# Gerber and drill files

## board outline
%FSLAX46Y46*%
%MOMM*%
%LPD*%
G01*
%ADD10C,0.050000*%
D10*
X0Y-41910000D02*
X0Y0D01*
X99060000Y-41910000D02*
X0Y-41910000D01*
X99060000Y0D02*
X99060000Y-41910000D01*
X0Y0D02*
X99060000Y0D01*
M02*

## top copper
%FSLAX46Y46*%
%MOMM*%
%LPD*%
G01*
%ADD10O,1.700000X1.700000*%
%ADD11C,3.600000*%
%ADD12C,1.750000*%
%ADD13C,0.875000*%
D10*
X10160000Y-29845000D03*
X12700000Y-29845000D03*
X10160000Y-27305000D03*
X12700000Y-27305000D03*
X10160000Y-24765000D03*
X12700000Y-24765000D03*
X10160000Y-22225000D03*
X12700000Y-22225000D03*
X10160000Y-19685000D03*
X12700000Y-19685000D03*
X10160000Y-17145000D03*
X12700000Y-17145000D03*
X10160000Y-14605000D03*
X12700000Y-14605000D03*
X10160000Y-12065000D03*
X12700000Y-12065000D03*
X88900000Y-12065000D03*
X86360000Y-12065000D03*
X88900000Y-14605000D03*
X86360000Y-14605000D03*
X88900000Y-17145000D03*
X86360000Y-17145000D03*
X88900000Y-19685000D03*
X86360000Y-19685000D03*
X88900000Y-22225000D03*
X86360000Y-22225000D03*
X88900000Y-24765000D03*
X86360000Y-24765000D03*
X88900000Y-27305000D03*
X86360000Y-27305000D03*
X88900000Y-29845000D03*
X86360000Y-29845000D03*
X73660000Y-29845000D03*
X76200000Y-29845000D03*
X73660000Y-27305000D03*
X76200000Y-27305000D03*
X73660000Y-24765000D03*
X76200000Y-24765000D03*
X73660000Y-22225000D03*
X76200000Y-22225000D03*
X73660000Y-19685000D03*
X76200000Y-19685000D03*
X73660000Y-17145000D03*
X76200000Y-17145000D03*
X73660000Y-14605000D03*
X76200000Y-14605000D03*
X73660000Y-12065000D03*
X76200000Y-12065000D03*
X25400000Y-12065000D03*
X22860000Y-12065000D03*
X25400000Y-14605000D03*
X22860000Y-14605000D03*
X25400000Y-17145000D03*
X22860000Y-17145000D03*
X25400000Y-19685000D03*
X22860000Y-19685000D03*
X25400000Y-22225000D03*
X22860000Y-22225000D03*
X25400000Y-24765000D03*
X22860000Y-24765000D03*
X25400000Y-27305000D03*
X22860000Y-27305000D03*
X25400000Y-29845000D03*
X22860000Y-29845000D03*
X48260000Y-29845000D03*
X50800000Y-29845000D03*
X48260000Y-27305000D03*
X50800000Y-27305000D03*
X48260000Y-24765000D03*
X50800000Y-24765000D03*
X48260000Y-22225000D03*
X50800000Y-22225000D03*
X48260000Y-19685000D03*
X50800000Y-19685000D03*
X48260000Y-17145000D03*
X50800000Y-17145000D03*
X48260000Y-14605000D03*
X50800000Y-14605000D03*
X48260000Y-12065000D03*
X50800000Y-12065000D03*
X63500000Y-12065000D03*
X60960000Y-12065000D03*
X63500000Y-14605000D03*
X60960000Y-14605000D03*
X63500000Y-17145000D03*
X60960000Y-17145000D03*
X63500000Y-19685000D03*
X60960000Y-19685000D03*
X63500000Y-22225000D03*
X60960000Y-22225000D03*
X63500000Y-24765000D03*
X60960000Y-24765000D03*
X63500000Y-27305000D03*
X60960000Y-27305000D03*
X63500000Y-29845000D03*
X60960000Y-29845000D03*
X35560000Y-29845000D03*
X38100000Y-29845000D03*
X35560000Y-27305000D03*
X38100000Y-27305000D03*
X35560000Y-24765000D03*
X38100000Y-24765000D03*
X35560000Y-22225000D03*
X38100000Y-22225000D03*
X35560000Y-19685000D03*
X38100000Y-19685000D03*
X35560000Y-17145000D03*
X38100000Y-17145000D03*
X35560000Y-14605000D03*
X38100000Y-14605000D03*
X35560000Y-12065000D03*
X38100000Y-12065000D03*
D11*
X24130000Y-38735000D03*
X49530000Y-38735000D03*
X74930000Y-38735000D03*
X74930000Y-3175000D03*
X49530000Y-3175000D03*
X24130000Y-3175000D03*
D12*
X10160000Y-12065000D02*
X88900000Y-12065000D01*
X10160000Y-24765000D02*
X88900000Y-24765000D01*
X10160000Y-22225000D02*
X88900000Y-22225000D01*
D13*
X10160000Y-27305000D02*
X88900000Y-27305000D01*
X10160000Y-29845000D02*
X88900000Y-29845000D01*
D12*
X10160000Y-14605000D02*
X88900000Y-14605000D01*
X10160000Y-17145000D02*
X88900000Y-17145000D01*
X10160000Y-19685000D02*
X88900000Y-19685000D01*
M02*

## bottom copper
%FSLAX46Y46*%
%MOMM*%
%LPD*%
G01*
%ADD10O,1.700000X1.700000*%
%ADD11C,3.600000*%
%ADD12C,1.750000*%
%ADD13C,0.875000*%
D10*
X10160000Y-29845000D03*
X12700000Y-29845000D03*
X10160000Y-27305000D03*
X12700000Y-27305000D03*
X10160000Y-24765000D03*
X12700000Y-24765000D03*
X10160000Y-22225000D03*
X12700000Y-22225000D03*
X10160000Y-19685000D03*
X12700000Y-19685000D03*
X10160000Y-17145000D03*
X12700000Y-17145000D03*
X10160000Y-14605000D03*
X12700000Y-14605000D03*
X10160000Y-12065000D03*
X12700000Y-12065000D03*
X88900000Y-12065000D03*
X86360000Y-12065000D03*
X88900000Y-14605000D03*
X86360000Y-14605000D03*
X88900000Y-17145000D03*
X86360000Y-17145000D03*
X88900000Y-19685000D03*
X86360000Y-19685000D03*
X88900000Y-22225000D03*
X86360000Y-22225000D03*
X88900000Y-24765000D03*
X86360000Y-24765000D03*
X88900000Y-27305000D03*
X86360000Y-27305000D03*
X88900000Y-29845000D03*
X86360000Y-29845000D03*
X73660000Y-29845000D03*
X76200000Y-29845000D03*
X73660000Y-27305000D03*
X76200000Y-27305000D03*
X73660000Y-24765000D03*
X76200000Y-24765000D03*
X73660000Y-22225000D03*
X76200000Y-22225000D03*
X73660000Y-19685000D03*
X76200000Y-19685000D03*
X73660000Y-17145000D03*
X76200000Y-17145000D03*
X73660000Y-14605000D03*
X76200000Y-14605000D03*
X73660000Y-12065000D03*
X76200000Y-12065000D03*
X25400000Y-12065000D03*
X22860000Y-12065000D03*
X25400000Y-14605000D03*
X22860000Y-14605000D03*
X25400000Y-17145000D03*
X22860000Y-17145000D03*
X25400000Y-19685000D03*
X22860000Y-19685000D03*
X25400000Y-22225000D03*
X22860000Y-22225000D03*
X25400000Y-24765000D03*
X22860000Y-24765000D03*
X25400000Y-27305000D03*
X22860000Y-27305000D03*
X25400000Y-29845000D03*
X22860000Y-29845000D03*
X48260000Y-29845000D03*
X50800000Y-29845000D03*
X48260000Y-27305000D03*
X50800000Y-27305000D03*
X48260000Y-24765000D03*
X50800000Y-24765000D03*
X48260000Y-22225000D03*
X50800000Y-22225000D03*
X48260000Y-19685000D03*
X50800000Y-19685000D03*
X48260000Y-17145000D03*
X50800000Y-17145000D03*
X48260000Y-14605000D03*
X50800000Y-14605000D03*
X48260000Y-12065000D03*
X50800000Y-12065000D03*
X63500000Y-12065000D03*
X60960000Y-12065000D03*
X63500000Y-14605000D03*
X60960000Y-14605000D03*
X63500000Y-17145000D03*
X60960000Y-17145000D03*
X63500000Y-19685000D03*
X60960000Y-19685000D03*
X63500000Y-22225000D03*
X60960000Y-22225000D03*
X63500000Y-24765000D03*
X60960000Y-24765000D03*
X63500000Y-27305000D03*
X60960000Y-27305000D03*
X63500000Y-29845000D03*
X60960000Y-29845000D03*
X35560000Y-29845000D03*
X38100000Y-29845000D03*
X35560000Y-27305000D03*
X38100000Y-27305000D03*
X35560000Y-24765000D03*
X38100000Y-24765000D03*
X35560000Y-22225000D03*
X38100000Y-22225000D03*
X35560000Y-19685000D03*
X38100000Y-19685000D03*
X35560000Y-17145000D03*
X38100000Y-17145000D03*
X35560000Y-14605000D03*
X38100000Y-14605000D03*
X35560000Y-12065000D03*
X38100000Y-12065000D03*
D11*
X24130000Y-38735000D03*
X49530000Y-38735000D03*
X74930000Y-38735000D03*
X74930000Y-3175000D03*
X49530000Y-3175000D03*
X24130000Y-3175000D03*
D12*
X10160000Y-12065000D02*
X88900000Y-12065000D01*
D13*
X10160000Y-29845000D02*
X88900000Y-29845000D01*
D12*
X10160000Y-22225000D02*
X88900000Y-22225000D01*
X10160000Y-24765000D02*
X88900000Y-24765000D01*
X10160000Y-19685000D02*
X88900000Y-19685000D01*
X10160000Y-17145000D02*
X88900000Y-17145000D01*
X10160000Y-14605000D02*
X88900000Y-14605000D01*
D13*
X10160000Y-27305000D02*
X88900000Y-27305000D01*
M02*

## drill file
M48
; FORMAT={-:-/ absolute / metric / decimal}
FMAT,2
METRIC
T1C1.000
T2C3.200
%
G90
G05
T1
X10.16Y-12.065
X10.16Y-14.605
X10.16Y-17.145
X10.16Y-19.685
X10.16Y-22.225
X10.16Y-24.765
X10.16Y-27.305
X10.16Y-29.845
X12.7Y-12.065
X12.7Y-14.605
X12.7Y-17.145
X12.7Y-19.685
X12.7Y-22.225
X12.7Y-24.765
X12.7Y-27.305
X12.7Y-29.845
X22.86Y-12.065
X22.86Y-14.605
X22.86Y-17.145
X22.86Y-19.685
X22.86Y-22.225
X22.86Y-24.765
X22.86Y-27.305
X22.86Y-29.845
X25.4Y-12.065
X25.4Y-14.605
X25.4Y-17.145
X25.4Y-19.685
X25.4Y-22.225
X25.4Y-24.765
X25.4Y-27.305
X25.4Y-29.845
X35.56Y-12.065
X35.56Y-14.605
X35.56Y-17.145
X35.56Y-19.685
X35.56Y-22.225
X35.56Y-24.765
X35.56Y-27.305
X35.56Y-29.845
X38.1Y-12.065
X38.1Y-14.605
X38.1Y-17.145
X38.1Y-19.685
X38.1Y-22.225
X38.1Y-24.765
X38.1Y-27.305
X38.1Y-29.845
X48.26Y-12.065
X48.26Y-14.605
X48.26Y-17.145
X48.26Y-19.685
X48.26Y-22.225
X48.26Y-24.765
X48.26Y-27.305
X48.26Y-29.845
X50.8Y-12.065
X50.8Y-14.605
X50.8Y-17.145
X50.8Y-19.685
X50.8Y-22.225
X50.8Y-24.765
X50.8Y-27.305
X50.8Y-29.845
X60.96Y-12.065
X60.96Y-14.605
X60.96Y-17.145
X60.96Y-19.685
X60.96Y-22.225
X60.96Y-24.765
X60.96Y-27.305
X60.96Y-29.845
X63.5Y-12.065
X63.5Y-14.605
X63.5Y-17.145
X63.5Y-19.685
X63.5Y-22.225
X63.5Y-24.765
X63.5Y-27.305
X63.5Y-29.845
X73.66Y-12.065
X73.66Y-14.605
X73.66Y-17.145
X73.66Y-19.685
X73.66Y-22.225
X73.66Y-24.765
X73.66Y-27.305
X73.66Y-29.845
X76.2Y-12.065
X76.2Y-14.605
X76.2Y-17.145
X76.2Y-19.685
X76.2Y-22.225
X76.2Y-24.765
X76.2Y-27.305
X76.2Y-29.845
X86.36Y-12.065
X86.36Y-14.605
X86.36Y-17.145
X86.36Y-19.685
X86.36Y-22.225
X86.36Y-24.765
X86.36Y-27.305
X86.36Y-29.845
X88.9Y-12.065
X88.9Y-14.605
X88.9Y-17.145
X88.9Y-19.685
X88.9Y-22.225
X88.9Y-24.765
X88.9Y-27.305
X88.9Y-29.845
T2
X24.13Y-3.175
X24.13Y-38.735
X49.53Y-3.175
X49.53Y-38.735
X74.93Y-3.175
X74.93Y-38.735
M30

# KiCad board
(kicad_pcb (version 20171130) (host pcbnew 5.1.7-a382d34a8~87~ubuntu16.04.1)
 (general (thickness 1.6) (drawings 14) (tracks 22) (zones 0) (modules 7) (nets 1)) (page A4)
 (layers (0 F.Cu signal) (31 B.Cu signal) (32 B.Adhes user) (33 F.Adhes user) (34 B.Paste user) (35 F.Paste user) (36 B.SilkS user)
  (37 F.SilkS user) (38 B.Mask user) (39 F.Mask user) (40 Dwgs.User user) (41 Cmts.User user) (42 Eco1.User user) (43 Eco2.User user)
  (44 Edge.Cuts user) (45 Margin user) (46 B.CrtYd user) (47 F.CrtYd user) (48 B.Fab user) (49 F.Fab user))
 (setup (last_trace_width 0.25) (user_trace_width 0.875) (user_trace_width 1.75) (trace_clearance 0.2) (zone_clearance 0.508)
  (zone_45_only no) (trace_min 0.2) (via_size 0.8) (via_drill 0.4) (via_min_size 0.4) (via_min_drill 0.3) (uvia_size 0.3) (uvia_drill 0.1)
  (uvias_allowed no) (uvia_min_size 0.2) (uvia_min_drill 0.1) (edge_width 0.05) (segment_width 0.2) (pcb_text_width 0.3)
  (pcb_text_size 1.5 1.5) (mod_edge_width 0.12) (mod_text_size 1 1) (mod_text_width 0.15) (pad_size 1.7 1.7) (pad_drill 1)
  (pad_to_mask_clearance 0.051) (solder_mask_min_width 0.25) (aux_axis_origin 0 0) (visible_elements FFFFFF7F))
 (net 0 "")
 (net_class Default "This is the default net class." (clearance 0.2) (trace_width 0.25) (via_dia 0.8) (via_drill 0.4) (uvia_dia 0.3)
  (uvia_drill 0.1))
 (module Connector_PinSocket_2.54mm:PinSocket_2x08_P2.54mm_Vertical (layer F.Cu) (at 12.7 12.065)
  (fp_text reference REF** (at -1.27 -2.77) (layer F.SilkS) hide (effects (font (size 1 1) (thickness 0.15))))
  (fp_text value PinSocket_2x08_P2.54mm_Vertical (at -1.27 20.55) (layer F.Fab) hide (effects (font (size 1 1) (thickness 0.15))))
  (pad 16 thru_hole oval (at -2.54 17.78) (size 1.7 1.7) (drill 1) (layers *.Cu *.Mask))
  (pad 15 thru_hole oval (at 0 17.78) (size 1.7 1.7) (drill 1) (layers *.Cu *.Mask))
  (pad 14 thru_hole oval (at -2.54 15.24) (size 1.7 1.7) (drill 1) (layers *.Cu *.Mask))
  (pad 13 thru_hole oval (at 0 15.24) (size 1.7 1.7) (drill 1) (layers *.Cu *.Mask))
  (pad 12 thru_hole oval (at -2.54 12.7) (size 1.7 1.7) (drill 1) (layers *.Cu *.Mask))
  (pad 11 thru_hole oval (at 0 12.7) (size 1.7 1.7) (drill 1) (layers *.Cu *.Mask))
  (pad 10 thru_hole oval (at -2.54 10.16) (size 1.7 1.7) (drill 1) (layers *.Cu *.Mask))
  (pad 9 thru_hole oval (at 0 10.16) (size 1.7 1.7) (drill 1) (layers *.Cu *.Mask))
  (pad 8 thru_hole oval (at -2.54 7.62) (size 1.7 1.7) (drill 1) (layers *.Cu *.Mask))
  (pad 7 thru_hole oval (at 0 7.62) (size 1.7 1.7) (drill 1) (layers *.Cu *.Mask))
  (pad 6 thru_hole oval (at -2.54 5.08) (size 1.7 1.7) (drill 1) (layers *.Cu *.Mask))
  (pad 5 thru_hole oval (at 0 5.08) (size 1.7 1.7) (drill 1) (layers *.Cu *.Mask))
  (pad 4 thru_hole oval (at -2.54 2.54) (size 1.7 1.7) (drill 1) (layers *.Cu *.Mask))
  (pad 3 thru_hole oval (at 0 2.54) (size 1.7 1.7) (drill 1) (layers *.Cu *.Mask))
  (pad 2 thru_hole oval (at -2.54 0) (size 1.7 1.7) (drill 1) (layers *.Cu *.Mask))
  (pad 1 thru_hole oval (at 0 0) (size 1.7 1.7) (drill 1) (layers *.Cu *.Mask)))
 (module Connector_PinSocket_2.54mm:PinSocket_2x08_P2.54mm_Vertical (layer F.Cu) (at 88.9 12.065)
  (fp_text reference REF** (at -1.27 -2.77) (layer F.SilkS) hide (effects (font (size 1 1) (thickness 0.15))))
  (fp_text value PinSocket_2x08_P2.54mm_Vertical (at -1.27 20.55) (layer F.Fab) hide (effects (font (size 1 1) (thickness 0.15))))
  (pad 1 thru_hole oval (at 0 0) (size 1.7 1.7) (drill 1) (layers *.Cu *.Mask))
  (pad 2 thru_hole oval (at -2.54 0) (size 1.7 1.7) (drill 1) (layers *.Cu *.Mask))
  (pad 3 thru_hole oval (at 0 2.54) (size 1.7 1.7) (drill 1) (layers *.Cu *.Mask))
  (pad 4 thru_hole oval (at -2.54 2.54) (size 1.7 1.7) (drill 1) (layers *.Cu *.Mask))
  (pad 5 thru_hole oval (at 0 5.08) (size 1.7 1.7) (drill 1) (layers *.Cu *.Mask))
  (pad 6 thru_hole oval (at -2.54 5.08) (size 1.7 1.7) (drill 1) (layers *.Cu *.Mask))
  (pad 7 thru_hole oval (at 0 7.62) (size 1.7 1.7) (drill 1) (layers *.Cu *.Mask))
  (pad 8 thru_hole oval (at -2.54 7.62) (size 1.7 1.7) (drill 1) (layers *.Cu *.Mask))
  (pad 9 thru_hole oval (at 0 10.16) (size 1.7 1.7) (drill 1) (layers *.Cu *.Mask))
  (pad 10 thru_hole oval (at -2.54 10.16) (size 1.7 1.7) (drill 1) (layers *.Cu *.Mask))
  (pad 11 thru_hole oval (at 0 12.7) (size 1.7 1.7) (drill 1) (layers *.Cu *.Mask))
  (pad 12 thru_hole oval (at -2.54 12.7) (size 1.7 1.7) (drill 1) (layers *.Cu *.Mask))
  (pad 13 thru_hole oval (at 0 15.24) (size 1.7 1.7) (drill 1) (layers *.Cu *.Mask))
  (pad 14 thru_hole oval (at -2.54 15.24) (size 1.7 1.7) (drill 1) (layers *.Cu *.Mask))
  (pad 15 thru_hole oval (at 0 17.78) (size 1.7 1.7) (drill 1) (layers *.Cu *.Mask))
  (pad 16 thru_hole oval (at -2.54 17.78) (size 1.7 1.7) (drill 1) (layers *.Cu *.Mask)))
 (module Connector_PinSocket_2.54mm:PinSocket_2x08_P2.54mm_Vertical (layer F.Cu) (at 76.2 12.065)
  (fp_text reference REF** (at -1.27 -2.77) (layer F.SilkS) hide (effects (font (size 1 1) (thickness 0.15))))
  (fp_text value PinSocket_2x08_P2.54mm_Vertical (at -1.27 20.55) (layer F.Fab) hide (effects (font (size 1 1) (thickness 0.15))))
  (pad 16 thru_hole oval (at -2.54 17.78) (size 1.7 1.7) (drill 1) (layers *.Cu *.Mask))
  (pad 15 thru_hole oval (at 0 17.78) (size 1.7 1.7) (drill 1) (layers *.Cu *.Mask))
  (pad 14 thru_hole oval (at -2.54 15.24) (size 1.7 1.7) (drill 1) (layers *.Cu *.Mask))
  (pad 13 thru_hole oval (at 0 15.24) (size 1.7 1.7) (drill 1) (layers *.Cu *.Mask))
  (pad 12 thru_hole oval (at -2.54 12.7) (size 1.7 1.7) (drill 1) (layers *.Cu *.Mask))
  (pad 11 thru_hole oval (at 0 12.7) (size 1.7 1.7) (drill 1) (layers *.Cu *.Mask))
  (pad 10 thru_hole oval (at -2.54 10.16) (size 1.7 1.7) (drill 1) (layers *.Cu *.Mask))
  (pad 9 thru_hole oval (at 0 10.16) (size 1.7 1.7) (drill 1) (layers *.Cu *.Mask))
  (pad 8 thru_hole oval (at -2.54 7.62) (size 1.7 1.7) (drill 1) (layers *.Cu *.Mask))
  (pad 7 thru_hole oval (at 0 7.62) (size 1.7 1.7) (drill 1) (layers *.Cu *.Mask))
  (pad 6 thru_hole oval (at -2.54 5.08) (size 1.7 1.7) (drill 1) (layers *.Cu *.Mask))
  (pad 5 thru_hole oval (at 0 5.08) (size 1.7 1.7) (drill 1) (layers *.Cu *.Mask))
  (pad 4 thru_hole oval (at -2.54 2.54) (size 1.7 1.7) (drill 1) (layers *.Cu *.Mask))
  (pad 3 thru_hole oval (at 0 2.54) (size 1.7 1.7) (drill 1) (layers *.Cu *.Mask))
  (pad 2 thru_hole oval (at -2.54 0) (size 1.7 1.7) (drill 1) (layers *.Cu *.Mask))
  (pad 1 thru_hole oval (at 0 0) (size 1.7 1.7) (drill 1) (layers *.Cu *.Mask)))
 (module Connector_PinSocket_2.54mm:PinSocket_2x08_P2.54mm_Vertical (layer F.Cu) (at 25.4 12.065)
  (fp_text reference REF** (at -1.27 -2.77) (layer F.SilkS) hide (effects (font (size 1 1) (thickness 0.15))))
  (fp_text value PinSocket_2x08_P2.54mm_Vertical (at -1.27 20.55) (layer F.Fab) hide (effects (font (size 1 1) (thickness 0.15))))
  (pad 1 thru_hole oval (at 0 0) (size 1.7 1.7) (drill 1) (layers *.Cu *.Mask))
  (pad 2 thru_hole oval (at -2.54 0) (size 1.7 1.7) (drill 1) (layers *.Cu *.Mask))
  (pad 3 thru_hole oval (at 0 2.54) (size 1.7 1.7) (drill 1) (layers *.Cu *.Mask))
  (pad 4 thru_hole oval (at -2.54 2.54) (size 1.7 1.7) (drill 1) (layers *.Cu *.Mask))
  (pad 5 thru_hole oval (at 0 5.08) (size 1.7 1.7) (drill 1) (layers *.Cu *.Mask))
  (pad 6 thru_hole oval (at -2.54 5.08) (size 1.7 1.7) (drill 1) (layers *.Cu *.Mask))
  (pad 7 thru_hole oval (at 0 7.62) (size 1.7 1.7) (drill 1) (layers *.Cu *.Mask))
  (pad 8 thru_hole oval (at -2.54 7.62) (size 1.7 1.7) (drill 1) (layers *.Cu *.Mask))
  (pad 9 thru_hole oval (at 0 10.16) (size 1.7 1.7) (drill 1) (layers *.Cu *.Mask))
  (pad 10 thru_hole oval (at -2.54 10.16) (size 1.7 1.7) (drill 1) (layers *.Cu *.Mask))
  (pad 11 thru_hole oval (at 0 12.7) (size 1.7 1.7) (drill 1) (layers *.Cu *.Mask))
  (pad 12 thru_hole oval (at -2.54 12.7) (size 1.7 1.7) (drill 1) (layers *.Cu *.Mask))
  (pad 13 thru_hole oval (at 0 15.24) (size 1.7 1.7) (drill 1) (layers *.Cu *.Mask))
  (pad 14 thru_hole oval (at -2.54 15.24) (size 1.7 1.7) (drill 1) (layers *.Cu *.Mask))
  (pad 15 thru_hole oval (at 0 17.78) (size 1.7 1.7) (drill 1) (layers *.Cu *.Mask))
  (pad 16 thru_hole oval (at -2.54 17.78) (size 1.7 1.7) (drill 1) (layers *.Cu *.Mask)))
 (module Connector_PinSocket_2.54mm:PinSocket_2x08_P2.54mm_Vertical (layer F.Cu) (at 50.8 12.065)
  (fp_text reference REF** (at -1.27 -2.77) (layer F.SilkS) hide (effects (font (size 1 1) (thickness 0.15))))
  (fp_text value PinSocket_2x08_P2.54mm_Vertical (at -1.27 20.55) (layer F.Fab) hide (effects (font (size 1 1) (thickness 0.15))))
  (pad 16 thru_hole oval (at -2.54 17.78) (size 1.7 1.7) (drill 1) (layers *.Cu *.Mask))
  (pad 15 thru_hole oval (at 0 17.78) (size 1.7 1.7) (drill 1) (layers *.Cu *.Mask))
  (pad 14 thru_hole oval (at -2.54 15.24) (size 1.7 1.7) (drill 1) (layers *.Cu *.Mask))
  (pad 13 thru_hole oval (at 0 15.24) (size 1.7 1.7) (drill 1) (layers *.Cu *.Mask))
  (pad 12 thru_hole oval (at -2.54 12.7) (size 1.7 1.7) (drill 1) (layers *.Cu *.Mask))
  (pad 11 thru_hole oval (at 0 12.7) (size 1.7 1.7) (drill 1) (layers *.Cu *.Mask))
  (pad 10 thru_hole oval (at -2.54 10.16) (size 1.7 1.7) (drill 1) (layers *.Cu *.Mask))
  (pad 9 thru_hole oval (at 0 10.16) (size 1.7 1.7) (drill 1) (layers *.Cu *.Mask))
  (pad 8 thru_hole oval (at -2.54 7.62) (size 1.7 1.7) (drill 1) (layers *.Cu *.Mask))
  (pad 7 thru_hole oval (at 0 7.62) (size 1.7 1.7) (drill 1) (layers *.Cu *.Mask))
  (pad 6 thru_hole oval (at -2.54 5.08) (size 1.7 1.7) (drill 1) (layers *.Cu *.Mask))
  (pad 5 thru_hole oval (at 0 5.08) (size 1.7 1.7) (drill 1) (layers *.Cu *.Mask))
  (pad 4 thru_hole oval (at -2.54 2.54) (size 1.7 1.7) (drill 1) (layers *.Cu *.Mask))
  (pad 3 thru_hole oval (at 0 2.54) (size 1.7 1.7) (drill 1) (layers *.Cu *.Mask))
  (pad 2 thru_hole oval (at -2.54 0) (size 1.7 1.7) (drill 1) (layers *.Cu *.Mask))
  (pad 1 thru_hole oval (at 0 0) (size 1.7 1.7) (drill 1) (layers *.Cu *.Mask)))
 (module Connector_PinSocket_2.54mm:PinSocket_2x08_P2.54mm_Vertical (layer F.Cu) (at 63.5 12.065)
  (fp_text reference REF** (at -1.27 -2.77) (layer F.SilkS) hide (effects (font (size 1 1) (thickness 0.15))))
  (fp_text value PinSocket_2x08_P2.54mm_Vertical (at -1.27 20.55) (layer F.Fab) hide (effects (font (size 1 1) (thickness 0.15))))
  (pad 1 thru_hole oval (at 0 0) (size 1.7 1.7) (drill 1) (layers *.Cu *.Mask))
  (pad 2 thru_hole oval (at -2.54 0) (size 1.7 1.7) (drill 1) (layers *.Cu *.Mask))
  (pad 3 thru_hole oval (at 0 2.54) (size 1.7 1.7) (drill 1) (layers *.Cu *.Mask))
  (pad 4 thru_hole oval (at -2.54 2.54) (size 1.7 1.7) (drill 1) (layers *.Cu *.Mask))
  (pad 5 thru_hole oval (at 0 5.08) (size 1.7 1.7) (drill 1) (layers *.Cu *.Mask))
  (pad 6 thru_hole oval (at -2.54 5.08) (size 1.7 1.7) (drill 1) (layers *.Cu *.Mask))
  (pad 7 thru_hole oval (at 0 7.62) (size 1.7 1.7) (drill 1) (layers *.Cu *.Mask))
  (pad 8 thru_hole oval (at -2.54 7.62) (size 1.7 1.7) (drill 1) (layers *.Cu *.Mask))
  (pad 9 thru_hole oval (at 0 10.16) (size 1.7 1.7) (drill 1) (layers *.Cu *.Mask))
  (pad 10 thru_hole oval (at -2.54 10.16) (size 1.7 1.7) (drill 1) (layers *.Cu *.Mask))
  (pad 11 thru_hole oval (at 0 12.7) (size 1.7 1.7) (drill 1) (layers *.Cu *.Mask))
  (pad 12 thru_hole oval (at -2.54 12.7) (size 1.7 1.7) (drill 1) (layers *.Cu *.Mask))
  (pad 13 thru_hole oval (at 0 15.24) (size 1.7 1.7) (drill 1) (layers *.Cu *.Mask))
  (pad 14 thru_hole oval (at -2.54 15.24) (size 1.7 1.7) (drill 1) (layers *.Cu *.Mask))
  (pad 15 thru_hole oval (at 0 17.78) (size 1.7 1.7) (drill 1) (layers *.Cu *.Mask))
  (pad 16 thru_hole oval (at -2.54 17.78) (size 1.7 1.7) (drill 1) (layers *.Cu *.Mask)))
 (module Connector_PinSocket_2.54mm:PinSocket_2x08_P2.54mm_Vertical (layer F.Cu) (at 38.1 12.065)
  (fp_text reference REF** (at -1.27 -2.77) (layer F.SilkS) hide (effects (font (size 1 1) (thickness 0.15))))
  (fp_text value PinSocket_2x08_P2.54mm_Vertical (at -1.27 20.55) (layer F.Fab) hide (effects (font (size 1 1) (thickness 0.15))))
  (pad 16 thru_hole oval (at -2.54 17.78) (size 1.7 1.7) (drill 1) (layers *.Cu *.Mask))
  (pad 15 thru_hole oval (at 0 17.78) (size 1.7 1.7) (drill 1) (layers *.Cu *.Mask))
  (pad 14 thru_hole oval (at -2.54 15.24) (size 1.7 1.7) (drill 1) (layers *.Cu *.Mask))
  (pad 13 thru_hole oval (at 0 15.24) (size 1.7 1.7) (drill 1) (layers *.Cu *.Mask))
  (pad 12 thru_hole oval (at -2.54 12.7) (size 1.7 1.7) (drill 1) (layers *.Cu *.Mask))
  (pad 11 thru_hole oval (at 0 12.7) (size 1.7 1.7) (drill 1) (layers *.Cu *.Mask))
  (pad 10 thru_hole oval (at -2.54 10.16) (size 1.7 1.7) (drill 1) (layers *.Cu *.Mask))
  (pad 9 thru_hole oval (at 0 10.16) (size 1.7 1.7) (drill 1) (layers *.Cu *.Mask))
  (pad 8 thru_hole oval (at -2.54 7.62) (size 1.7 1.7) (drill 1) (layers *.Cu *.Mask))
  (pad 7 thru_hole oval (at 0 7.62) (size 1.7 1.7) (drill 1) (layers *.Cu *.Mask))
  (pad 6 thru_hole oval (at -2.54 5.08) (size 1.7 1.7) (drill 1) (layers *.Cu *.Mask))
  (pad 5 thru_hole oval (at 0 5.08) (size 1.7 1.7) (drill 1) (layers *.Cu *.Mask))
  (pad 4 thru_hole oval (at -2.54 2.54) (size 1.7 1.7) (drill 1) (layers *.Cu *.Mask))
  (pad 3 thru_hole oval (at 0 2.54) (size 1.7 1.7) (drill 1) (layers *.Cu *.Mask))
  (pad 2 thru_hole oval (at -2.54 0) (size 1.7 1.7) (drill 1) (layers *.Cu *.Mask))
  (pad 1 thru_hole oval (at 0 0) (size 1.7 1.7) (drill 1) (layers *.Cu *.Mask)))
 (gr_line (start 0 41.91) (end 0 0) (layer Edge.Cuts) (width 0.05))
 (gr_line (start 99.06 41.91) (end 0 41.91) (layer Edge.Cuts) (width 0.05))
 (gr_line (start 99.06 0) (end 99.06 41.91) (layer Edge.Cuts) (width 0.05))
 (gr_line (start 0 0) (end 99.06 0) (layer Edge.Cuts) (width 0.05))
 (via (at 24.13 38.735) (size 3.6) (drill 3.2) (layers F.Cu B.Cu) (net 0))
 (via (at 49.53 38.735) (size 3.6) (drill 3.2) (layers F.Cu B.Cu) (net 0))
 (via (at 74.93 38.735) (size 3.6) (drill 3.2) (layers F.Cu B.Cu) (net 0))
 (via (at 74.93 3.175) (size 3.6) (drill 3.2) (layers F.Cu B.Cu) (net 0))
 (via (at 49.53 3.175) (size 3.6) (drill 3.2) (layers F.Cu B.Cu) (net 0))
 (via (at 24.13 3.175) (size 3.6) (drill 3.2) (layers F.Cu B.Cu) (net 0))
 (segment (start 10.16 12.065) (end 88.9 12.065) (width 1.75) (layer F.Cu) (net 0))
 (segment (start 10.16 24.765) (end 88.9 24.765) (width 1.75) (layer F.Cu) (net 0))
 (segment (start 10.16 22.225) (end 88.9 22.225) (width 1.75) (layer F.Cu) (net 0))
 (segment (start 10.16 27.305) (end 88.9 27.305) (width 0.875) (layer F.Cu) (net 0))
 (segment (start 10.16 29.845) (end 88.9 29.845) (width 0.875) (layer F.Cu) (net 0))
 (segment (start 10.16 14.605) (end 88.9 14.605) (width 1.75) (layer F.Cu) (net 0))
 (segment (start 10.16 17.145) (end 88.9 17.145) (width 1.75) (layer F.Cu) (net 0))
 (segment (start 10.16 19.685) (end 88.9 19.685) (width 1.75) (layer F.Cu) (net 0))
 (segment (start 10.16 12.065) (end 88.9 12.065) (width 1.75) (layer B.Cu) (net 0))
 (segment (start 10.16 29.845) (end 88.9 29.845) (width 0.875) (layer B.Cu) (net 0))
 (segment (start 10.16 22.225) (end 88.9 22.225) (width 1.75) (layer B.Cu) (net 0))
 (segment (start 10.16 24.765) (end 88.9 24.765) (width 1.75) (layer B.Cu) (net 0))
 (segment (start 10.16 19.685) (end 88.9 19.685) (width 1.75) (layer B.Cu) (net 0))
 (segment (start 10.16 17.145) (end 88.9 17.145) (width 1.75) (layer B.Cu) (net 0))
 (segment (start 10.16 14.605) (end 88.9 14.605) (width 1.75) (layer B.Cu) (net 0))
 (segment (start 10.16 27.305) (end 88.9 27.305) (width 0.875) (layer B.Cu) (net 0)))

